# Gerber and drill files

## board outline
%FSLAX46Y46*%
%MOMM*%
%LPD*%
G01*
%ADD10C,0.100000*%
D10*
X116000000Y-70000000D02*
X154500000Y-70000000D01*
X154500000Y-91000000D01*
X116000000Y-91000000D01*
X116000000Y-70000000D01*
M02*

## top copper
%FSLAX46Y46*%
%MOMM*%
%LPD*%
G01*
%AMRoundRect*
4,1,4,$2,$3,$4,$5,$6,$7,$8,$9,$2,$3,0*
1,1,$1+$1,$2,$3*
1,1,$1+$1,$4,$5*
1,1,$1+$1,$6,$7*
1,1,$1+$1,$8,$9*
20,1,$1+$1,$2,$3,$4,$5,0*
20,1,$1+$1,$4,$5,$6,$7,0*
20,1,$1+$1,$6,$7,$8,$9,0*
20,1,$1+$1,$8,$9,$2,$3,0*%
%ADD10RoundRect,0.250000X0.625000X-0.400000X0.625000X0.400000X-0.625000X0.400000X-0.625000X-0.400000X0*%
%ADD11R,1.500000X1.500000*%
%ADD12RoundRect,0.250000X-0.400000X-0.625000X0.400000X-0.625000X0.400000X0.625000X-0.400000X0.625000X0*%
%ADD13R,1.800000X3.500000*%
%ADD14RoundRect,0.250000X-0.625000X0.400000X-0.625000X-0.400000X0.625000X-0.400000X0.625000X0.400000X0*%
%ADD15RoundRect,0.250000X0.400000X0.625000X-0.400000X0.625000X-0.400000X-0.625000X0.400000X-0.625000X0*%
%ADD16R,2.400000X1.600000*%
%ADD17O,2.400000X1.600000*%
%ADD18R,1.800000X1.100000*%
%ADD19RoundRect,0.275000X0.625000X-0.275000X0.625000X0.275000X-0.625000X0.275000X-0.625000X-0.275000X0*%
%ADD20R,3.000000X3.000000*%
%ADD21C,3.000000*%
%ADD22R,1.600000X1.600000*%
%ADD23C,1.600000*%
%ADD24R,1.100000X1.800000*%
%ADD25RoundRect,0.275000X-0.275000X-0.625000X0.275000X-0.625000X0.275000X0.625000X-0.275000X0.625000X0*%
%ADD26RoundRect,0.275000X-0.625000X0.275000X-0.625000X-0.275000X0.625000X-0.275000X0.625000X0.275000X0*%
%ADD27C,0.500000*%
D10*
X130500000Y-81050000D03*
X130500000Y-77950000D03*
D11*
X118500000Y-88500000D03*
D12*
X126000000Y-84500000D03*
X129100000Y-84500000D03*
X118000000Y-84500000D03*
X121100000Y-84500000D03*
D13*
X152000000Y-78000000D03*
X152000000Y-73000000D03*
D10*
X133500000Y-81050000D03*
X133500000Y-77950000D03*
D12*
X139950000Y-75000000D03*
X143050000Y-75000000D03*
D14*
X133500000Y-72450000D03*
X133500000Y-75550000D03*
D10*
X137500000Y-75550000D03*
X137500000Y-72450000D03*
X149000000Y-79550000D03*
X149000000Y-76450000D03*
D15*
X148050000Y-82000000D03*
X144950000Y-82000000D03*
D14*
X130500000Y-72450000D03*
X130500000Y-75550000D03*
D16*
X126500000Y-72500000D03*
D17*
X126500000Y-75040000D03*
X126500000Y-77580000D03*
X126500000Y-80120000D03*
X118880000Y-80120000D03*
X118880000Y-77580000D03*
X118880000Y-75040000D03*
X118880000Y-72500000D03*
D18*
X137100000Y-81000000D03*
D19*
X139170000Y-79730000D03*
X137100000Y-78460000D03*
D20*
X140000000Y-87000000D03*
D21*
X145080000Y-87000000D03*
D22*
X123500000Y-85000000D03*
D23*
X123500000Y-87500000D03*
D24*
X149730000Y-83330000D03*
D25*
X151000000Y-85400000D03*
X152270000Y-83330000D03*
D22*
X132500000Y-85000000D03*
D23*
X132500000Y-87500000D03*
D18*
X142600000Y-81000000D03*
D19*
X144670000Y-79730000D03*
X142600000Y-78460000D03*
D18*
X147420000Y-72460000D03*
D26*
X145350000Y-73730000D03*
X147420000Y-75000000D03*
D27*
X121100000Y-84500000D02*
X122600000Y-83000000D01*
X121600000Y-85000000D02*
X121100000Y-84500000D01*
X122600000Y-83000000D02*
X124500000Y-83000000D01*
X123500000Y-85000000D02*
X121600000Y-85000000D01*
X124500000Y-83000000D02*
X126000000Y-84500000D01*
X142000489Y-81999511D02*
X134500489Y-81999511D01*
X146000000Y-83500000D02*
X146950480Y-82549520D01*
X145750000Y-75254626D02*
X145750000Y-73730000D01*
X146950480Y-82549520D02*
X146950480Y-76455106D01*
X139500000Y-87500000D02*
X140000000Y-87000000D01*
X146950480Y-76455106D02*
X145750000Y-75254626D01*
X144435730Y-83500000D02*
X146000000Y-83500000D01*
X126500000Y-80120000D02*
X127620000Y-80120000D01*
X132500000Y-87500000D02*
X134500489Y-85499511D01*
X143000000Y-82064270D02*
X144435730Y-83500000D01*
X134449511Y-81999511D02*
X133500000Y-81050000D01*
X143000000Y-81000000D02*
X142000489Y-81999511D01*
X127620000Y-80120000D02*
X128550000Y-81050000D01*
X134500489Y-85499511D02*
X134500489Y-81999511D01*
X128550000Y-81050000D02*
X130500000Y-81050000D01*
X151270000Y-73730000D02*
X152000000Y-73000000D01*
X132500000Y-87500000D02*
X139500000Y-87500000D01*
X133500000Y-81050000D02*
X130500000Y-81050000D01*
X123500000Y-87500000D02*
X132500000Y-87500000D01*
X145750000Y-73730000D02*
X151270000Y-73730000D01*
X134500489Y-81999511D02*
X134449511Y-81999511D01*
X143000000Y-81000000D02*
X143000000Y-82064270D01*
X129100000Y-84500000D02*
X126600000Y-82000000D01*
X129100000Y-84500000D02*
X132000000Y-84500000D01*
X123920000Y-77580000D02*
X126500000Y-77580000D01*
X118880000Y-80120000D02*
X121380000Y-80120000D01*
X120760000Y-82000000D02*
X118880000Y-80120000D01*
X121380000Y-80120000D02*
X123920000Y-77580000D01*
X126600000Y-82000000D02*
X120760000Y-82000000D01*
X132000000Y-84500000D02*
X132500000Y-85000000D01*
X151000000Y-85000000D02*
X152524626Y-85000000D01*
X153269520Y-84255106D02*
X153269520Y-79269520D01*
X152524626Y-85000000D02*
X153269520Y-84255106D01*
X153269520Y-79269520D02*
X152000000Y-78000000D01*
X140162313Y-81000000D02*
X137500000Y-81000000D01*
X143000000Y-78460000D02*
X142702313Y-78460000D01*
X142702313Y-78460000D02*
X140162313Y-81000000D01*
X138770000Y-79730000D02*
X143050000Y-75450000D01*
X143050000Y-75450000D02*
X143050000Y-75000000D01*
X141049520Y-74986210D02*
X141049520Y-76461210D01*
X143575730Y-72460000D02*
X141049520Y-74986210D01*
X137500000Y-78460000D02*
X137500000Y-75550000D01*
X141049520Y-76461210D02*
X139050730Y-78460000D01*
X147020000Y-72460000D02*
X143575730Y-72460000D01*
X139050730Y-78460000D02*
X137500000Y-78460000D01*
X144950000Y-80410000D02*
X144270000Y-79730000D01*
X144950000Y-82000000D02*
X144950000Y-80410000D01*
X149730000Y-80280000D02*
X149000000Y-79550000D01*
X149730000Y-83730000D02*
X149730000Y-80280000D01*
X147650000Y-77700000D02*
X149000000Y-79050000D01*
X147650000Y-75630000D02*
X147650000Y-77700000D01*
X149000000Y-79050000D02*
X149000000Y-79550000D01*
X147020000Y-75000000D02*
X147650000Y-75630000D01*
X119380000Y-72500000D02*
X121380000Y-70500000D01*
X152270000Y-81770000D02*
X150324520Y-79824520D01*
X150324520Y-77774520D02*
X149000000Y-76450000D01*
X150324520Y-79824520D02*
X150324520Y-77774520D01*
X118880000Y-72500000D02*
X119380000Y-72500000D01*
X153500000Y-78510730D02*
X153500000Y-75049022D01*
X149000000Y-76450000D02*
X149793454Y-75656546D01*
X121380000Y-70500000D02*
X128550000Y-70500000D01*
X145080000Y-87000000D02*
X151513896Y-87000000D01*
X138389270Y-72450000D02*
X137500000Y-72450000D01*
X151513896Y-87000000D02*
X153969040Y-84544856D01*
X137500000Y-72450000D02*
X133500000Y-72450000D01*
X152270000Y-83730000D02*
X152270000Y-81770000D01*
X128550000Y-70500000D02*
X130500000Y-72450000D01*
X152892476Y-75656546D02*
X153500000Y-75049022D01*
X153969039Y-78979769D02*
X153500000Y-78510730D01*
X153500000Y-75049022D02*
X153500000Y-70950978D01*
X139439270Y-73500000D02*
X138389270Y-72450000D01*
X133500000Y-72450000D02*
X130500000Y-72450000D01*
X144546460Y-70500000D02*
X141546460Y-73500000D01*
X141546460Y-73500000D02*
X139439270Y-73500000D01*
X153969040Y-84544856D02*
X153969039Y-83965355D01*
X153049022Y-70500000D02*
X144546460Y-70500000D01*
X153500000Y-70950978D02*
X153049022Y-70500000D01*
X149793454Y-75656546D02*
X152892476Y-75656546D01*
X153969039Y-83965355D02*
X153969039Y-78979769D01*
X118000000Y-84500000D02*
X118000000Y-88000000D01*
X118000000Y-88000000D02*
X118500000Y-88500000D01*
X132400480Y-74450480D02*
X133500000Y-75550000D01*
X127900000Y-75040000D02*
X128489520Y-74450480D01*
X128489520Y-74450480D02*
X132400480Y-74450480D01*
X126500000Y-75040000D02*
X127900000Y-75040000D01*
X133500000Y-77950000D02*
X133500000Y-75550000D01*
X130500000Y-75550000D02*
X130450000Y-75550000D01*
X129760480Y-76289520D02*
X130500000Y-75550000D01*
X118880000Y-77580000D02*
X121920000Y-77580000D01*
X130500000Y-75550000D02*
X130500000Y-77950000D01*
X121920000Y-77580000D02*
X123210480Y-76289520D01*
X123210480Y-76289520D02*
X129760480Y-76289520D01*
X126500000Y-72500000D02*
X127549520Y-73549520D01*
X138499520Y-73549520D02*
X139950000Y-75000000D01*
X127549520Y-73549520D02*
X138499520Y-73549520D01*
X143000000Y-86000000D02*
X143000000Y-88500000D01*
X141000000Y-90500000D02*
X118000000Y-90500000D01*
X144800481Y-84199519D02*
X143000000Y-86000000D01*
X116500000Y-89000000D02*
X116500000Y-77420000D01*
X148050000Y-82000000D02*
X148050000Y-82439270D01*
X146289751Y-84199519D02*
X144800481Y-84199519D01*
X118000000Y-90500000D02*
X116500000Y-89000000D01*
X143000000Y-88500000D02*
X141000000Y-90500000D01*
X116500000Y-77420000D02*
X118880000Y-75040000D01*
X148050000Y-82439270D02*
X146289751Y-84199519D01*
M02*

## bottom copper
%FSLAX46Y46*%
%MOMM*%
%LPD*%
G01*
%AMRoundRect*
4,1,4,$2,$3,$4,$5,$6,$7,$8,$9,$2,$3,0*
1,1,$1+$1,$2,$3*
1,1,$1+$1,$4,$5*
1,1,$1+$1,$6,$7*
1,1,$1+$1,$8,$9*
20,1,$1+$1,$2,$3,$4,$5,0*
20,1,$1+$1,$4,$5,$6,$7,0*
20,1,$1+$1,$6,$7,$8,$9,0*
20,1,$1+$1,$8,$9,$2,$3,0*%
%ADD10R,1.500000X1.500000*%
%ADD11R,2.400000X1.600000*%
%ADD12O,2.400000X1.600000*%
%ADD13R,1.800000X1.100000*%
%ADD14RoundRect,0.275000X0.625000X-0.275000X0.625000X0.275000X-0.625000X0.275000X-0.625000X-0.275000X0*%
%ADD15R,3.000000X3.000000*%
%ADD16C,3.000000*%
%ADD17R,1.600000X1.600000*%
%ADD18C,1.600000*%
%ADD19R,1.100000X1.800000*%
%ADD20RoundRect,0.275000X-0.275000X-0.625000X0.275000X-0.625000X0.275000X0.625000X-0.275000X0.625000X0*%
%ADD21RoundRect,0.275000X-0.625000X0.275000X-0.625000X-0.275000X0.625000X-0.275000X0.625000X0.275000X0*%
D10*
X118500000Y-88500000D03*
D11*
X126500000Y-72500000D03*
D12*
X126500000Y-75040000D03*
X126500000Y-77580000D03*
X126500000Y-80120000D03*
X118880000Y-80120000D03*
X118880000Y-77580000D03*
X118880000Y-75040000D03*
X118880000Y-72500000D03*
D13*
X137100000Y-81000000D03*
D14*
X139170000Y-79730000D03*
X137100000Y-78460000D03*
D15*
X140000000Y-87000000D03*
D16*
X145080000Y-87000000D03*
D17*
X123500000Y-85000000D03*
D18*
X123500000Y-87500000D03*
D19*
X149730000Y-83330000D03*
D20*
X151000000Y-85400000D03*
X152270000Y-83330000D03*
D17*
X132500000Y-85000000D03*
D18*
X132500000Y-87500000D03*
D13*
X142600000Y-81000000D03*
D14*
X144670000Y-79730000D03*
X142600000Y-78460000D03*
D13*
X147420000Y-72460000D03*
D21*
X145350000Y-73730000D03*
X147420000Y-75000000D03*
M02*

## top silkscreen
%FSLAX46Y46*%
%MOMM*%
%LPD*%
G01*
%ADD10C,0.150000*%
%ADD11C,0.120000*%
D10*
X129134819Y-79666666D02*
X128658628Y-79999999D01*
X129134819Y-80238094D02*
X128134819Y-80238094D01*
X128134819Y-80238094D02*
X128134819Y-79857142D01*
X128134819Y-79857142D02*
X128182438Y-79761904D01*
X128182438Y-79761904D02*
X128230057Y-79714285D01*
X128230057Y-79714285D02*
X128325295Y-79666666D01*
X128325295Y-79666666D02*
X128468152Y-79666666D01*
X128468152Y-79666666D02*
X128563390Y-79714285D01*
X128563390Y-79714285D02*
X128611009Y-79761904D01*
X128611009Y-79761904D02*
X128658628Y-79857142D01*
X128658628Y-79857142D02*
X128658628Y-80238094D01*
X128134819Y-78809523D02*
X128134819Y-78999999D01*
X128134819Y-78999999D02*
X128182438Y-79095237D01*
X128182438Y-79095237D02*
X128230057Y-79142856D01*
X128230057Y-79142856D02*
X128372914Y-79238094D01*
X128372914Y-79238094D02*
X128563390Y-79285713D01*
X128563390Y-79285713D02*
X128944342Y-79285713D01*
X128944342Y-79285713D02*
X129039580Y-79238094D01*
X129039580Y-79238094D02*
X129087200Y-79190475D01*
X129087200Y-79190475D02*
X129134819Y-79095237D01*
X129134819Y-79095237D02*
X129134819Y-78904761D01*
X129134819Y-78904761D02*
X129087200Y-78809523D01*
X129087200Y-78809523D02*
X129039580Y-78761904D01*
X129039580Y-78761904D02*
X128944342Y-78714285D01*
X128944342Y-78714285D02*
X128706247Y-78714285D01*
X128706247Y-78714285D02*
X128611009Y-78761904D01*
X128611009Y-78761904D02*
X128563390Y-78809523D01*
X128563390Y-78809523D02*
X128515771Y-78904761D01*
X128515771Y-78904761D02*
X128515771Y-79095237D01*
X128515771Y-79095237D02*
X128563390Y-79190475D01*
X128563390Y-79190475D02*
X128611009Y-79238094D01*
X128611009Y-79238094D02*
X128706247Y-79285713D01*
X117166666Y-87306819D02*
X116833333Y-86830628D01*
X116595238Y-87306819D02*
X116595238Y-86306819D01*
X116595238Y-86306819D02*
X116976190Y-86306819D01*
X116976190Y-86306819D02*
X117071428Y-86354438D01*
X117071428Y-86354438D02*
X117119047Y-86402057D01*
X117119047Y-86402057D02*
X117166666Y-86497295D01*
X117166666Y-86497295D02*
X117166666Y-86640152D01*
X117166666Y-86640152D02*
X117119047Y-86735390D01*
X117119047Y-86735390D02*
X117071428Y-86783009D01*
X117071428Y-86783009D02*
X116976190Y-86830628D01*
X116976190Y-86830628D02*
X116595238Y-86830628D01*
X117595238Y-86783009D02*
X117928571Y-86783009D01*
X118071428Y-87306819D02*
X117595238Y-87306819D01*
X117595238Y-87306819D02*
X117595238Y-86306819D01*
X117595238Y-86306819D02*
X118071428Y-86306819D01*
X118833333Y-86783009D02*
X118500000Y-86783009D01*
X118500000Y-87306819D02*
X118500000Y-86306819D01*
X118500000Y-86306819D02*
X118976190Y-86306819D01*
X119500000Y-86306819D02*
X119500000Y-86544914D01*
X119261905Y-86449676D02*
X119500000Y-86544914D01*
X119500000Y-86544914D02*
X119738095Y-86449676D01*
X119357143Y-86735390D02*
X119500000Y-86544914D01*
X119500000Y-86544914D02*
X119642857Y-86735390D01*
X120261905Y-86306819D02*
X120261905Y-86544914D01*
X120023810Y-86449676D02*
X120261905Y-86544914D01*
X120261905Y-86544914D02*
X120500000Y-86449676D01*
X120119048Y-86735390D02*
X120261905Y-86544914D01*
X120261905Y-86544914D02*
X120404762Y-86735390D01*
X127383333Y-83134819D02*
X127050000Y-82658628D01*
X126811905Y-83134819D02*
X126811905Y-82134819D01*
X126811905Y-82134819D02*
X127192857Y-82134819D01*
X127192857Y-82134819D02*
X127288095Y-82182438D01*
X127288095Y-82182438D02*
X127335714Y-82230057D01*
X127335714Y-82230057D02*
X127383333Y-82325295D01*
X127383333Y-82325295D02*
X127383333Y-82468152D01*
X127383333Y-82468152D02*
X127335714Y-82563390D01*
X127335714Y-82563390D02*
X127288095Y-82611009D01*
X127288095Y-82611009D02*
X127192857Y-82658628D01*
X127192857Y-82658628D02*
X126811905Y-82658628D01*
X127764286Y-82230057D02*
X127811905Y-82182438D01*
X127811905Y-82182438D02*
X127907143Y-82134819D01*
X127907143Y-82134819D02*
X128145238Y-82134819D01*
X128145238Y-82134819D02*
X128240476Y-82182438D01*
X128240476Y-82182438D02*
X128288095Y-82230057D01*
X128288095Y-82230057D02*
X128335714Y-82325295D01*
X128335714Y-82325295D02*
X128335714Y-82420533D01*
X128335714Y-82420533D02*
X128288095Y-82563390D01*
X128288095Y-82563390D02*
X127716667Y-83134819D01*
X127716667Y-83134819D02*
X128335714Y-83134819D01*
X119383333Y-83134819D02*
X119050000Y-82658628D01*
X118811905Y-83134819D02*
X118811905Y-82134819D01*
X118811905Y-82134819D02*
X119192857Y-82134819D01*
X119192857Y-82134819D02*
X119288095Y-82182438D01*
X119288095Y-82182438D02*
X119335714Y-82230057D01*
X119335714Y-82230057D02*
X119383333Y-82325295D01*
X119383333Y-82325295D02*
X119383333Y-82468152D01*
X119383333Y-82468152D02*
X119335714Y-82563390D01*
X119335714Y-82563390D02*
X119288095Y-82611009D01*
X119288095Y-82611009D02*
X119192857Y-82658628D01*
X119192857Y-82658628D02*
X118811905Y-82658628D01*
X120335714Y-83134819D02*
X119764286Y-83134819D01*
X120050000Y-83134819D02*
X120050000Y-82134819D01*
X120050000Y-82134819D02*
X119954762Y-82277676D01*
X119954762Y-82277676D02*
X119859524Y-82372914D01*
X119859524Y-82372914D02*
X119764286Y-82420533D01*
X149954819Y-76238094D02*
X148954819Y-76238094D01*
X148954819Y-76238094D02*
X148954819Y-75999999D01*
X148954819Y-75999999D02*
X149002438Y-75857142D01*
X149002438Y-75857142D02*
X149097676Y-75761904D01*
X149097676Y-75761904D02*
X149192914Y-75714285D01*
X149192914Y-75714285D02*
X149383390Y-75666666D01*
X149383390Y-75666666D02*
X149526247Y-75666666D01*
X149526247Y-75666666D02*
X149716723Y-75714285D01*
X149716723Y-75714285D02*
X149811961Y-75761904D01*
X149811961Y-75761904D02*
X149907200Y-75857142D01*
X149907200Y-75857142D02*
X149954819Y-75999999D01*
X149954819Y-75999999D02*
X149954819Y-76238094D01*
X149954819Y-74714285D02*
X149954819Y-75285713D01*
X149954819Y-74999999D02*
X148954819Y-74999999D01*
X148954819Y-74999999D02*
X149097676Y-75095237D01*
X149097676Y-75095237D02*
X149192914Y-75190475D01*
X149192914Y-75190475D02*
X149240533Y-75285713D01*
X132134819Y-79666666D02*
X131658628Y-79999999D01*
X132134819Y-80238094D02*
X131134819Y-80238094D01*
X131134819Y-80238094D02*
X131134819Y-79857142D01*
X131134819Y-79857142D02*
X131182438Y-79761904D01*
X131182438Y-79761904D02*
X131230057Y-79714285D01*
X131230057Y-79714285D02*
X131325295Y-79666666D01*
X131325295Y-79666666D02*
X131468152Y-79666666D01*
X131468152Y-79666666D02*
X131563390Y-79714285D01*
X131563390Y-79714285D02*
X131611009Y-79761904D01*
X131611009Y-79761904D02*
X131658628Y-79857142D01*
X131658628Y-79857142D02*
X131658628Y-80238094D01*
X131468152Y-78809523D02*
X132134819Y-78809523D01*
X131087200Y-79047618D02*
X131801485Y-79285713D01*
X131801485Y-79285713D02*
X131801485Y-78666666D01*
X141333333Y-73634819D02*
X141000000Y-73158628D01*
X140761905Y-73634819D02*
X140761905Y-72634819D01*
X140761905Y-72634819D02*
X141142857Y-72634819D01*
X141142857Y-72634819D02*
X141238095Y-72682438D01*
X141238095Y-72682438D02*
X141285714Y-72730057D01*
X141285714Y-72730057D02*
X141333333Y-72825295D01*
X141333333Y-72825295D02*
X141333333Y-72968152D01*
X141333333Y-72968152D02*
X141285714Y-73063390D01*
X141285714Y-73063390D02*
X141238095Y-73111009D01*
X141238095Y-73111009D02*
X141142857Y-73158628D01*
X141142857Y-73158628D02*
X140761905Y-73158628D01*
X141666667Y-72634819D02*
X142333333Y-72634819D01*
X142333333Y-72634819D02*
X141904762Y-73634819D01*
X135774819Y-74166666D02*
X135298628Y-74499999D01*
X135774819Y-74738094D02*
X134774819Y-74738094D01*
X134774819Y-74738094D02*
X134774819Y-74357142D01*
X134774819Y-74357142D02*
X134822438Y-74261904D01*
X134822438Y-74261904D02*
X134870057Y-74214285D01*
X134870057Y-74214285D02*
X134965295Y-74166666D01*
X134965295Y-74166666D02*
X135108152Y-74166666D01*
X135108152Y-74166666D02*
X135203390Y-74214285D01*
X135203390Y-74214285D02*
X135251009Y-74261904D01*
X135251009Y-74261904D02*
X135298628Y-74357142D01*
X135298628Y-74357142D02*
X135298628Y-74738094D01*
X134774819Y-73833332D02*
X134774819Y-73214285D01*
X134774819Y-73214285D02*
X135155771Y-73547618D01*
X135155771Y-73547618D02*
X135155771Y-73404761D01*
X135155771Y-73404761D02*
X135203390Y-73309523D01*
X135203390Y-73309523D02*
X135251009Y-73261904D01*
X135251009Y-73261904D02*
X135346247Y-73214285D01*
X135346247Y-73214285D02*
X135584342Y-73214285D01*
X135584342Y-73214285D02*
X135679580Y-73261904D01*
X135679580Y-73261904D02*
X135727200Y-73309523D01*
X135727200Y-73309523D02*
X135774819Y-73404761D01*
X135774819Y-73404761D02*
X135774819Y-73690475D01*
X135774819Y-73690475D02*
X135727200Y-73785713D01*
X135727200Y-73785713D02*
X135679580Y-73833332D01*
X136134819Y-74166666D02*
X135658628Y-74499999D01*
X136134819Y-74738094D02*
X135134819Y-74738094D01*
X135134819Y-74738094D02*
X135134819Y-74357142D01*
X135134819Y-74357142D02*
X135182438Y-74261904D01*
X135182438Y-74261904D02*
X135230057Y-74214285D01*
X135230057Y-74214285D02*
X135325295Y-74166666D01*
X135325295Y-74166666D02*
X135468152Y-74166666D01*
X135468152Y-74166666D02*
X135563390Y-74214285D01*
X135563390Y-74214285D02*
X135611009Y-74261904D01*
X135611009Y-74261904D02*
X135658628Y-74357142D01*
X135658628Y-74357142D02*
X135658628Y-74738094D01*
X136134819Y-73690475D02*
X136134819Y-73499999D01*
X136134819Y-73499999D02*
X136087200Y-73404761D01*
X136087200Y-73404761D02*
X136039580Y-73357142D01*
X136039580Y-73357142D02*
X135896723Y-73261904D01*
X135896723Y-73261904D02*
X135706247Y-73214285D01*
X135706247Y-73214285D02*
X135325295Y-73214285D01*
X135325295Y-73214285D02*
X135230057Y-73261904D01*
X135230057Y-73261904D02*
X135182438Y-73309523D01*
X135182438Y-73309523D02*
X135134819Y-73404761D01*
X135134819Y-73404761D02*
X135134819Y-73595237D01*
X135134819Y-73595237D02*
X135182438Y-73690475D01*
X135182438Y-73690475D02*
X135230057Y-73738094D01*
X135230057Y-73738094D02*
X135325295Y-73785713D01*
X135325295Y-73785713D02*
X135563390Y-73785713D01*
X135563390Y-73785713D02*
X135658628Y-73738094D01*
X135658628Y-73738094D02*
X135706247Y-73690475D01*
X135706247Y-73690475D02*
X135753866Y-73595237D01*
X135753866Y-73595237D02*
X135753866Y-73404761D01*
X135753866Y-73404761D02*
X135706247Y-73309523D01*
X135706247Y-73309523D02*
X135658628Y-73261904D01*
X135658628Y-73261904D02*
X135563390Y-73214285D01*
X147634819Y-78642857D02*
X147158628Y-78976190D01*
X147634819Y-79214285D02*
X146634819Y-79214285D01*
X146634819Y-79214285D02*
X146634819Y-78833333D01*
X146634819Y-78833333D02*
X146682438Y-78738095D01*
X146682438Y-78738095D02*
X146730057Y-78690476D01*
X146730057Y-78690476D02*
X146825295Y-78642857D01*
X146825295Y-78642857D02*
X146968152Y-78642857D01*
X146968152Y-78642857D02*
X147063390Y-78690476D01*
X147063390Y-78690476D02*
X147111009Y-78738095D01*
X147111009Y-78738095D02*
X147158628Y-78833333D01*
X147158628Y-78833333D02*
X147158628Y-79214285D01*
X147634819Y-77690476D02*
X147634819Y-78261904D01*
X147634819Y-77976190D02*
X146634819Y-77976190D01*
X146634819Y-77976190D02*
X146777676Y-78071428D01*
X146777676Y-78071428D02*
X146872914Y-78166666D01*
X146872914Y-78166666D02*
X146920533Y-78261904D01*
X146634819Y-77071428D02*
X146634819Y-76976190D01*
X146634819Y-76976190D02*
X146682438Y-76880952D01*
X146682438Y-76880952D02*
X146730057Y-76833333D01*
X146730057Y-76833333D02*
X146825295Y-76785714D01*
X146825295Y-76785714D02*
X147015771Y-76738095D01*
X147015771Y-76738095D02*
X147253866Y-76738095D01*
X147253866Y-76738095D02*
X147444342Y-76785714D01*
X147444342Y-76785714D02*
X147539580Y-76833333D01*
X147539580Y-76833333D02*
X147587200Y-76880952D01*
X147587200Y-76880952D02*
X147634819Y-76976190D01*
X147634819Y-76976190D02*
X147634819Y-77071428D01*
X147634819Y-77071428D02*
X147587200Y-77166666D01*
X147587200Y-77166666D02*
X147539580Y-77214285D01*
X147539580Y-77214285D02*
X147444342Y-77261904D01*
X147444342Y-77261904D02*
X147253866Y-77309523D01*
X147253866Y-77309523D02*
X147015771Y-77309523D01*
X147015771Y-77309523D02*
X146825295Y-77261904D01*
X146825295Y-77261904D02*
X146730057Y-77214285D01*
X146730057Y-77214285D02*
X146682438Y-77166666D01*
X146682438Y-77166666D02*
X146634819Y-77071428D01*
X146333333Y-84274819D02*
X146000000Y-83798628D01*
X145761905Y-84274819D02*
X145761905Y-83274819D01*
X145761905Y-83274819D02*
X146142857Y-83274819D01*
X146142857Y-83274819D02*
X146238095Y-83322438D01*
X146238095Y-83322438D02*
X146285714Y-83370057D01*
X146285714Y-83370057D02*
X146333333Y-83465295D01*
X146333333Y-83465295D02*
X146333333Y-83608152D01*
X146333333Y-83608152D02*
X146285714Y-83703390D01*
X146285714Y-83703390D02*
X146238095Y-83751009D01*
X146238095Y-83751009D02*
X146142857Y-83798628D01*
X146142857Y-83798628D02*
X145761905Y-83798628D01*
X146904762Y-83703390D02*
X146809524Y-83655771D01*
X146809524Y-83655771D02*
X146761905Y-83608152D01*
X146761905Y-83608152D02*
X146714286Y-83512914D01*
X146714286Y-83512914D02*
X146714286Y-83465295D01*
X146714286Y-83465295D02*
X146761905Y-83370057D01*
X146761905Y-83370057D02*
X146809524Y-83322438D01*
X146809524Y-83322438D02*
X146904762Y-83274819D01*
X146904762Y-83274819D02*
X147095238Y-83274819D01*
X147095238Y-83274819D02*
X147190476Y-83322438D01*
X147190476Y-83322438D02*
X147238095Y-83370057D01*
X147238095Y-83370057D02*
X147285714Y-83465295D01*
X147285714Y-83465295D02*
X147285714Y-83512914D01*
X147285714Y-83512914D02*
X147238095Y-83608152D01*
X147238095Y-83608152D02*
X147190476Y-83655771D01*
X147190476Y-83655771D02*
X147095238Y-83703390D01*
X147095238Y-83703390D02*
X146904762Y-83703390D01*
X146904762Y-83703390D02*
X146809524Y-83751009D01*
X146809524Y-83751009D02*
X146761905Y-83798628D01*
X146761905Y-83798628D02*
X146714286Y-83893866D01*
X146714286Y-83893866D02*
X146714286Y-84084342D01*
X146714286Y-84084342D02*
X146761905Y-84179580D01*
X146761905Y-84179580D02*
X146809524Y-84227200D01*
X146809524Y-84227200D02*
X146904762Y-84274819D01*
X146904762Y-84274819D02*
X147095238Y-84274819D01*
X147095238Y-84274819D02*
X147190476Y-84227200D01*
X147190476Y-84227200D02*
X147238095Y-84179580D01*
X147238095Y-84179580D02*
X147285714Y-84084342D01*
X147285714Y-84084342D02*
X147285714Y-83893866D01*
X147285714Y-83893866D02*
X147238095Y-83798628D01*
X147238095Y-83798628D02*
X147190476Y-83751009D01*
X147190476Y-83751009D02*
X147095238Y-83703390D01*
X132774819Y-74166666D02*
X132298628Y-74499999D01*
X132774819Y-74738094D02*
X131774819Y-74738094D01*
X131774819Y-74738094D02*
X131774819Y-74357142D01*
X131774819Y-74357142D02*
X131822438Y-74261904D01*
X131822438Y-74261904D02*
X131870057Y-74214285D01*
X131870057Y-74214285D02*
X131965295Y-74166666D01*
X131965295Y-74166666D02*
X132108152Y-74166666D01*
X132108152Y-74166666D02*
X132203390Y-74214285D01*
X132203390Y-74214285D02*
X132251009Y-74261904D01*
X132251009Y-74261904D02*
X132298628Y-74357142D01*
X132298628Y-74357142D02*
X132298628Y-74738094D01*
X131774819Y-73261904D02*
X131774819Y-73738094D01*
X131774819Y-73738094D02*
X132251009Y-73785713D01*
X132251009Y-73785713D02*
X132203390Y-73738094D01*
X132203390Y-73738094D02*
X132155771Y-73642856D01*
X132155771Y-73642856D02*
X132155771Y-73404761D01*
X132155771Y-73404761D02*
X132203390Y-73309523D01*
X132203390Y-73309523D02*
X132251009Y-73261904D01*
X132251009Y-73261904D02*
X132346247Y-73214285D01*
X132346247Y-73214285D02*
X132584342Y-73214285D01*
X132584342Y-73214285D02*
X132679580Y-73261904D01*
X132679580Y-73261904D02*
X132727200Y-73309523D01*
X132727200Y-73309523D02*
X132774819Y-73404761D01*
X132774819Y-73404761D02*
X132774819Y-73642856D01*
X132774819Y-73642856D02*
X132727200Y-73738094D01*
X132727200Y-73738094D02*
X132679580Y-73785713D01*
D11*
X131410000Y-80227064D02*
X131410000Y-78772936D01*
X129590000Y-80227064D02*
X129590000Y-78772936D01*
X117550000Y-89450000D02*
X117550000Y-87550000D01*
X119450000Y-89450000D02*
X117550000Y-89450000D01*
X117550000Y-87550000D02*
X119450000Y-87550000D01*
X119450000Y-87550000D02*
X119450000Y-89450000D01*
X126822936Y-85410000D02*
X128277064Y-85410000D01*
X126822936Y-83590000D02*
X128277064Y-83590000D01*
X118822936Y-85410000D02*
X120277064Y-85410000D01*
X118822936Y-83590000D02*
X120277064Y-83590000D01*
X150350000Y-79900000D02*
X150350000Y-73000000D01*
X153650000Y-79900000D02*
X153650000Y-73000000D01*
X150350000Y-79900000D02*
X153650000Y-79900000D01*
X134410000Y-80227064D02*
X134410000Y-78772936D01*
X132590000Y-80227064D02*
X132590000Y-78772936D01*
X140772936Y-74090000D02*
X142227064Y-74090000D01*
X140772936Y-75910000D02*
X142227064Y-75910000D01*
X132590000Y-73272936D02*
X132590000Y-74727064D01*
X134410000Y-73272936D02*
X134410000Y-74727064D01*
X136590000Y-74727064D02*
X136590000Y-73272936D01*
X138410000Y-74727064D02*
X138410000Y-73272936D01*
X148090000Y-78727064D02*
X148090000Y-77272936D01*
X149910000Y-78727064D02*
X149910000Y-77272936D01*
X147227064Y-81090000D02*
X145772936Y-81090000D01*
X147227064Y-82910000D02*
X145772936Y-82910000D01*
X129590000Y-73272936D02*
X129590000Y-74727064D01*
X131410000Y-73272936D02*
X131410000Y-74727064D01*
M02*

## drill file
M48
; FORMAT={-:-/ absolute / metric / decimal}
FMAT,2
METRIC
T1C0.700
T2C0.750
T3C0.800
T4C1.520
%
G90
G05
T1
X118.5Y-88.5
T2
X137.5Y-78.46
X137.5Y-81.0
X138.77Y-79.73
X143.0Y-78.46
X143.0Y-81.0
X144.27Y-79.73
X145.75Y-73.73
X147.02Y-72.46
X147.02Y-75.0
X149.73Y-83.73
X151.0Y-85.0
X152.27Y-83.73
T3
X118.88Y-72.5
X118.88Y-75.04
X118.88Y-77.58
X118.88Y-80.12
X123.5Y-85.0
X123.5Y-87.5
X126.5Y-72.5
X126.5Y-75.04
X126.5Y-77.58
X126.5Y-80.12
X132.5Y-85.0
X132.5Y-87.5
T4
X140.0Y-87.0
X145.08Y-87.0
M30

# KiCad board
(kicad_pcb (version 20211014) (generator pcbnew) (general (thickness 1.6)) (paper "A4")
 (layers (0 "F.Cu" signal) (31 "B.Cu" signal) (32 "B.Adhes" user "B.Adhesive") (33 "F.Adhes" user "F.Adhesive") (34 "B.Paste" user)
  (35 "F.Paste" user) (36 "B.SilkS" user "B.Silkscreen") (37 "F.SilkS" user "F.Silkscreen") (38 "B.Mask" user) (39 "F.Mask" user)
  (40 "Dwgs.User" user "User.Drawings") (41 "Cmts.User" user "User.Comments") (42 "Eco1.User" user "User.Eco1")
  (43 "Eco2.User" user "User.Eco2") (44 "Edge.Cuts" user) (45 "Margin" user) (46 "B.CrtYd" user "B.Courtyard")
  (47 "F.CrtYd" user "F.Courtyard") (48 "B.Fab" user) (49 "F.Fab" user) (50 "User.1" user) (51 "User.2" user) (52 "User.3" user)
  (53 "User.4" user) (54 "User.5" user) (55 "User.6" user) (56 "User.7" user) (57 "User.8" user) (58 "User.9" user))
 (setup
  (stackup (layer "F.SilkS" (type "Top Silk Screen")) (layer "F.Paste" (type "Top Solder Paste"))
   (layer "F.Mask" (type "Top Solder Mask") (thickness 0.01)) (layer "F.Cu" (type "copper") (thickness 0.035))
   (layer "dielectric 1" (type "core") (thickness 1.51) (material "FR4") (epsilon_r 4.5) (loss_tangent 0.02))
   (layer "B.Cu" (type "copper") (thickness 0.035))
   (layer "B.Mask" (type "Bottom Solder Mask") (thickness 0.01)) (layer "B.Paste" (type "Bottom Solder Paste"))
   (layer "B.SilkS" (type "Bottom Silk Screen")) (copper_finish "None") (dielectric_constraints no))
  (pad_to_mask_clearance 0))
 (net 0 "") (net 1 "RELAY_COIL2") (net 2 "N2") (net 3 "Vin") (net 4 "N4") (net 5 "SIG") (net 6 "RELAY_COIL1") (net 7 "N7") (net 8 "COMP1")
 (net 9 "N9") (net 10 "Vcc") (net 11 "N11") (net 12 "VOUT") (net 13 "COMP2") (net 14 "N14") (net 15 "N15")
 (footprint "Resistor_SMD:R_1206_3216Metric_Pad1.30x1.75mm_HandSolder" (layer "F.Cu") (at 130.5 79.5 90)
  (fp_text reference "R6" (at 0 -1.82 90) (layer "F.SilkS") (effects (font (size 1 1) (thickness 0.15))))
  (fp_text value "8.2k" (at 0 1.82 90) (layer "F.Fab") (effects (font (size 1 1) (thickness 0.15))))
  (fp_line (start -0.727064 0.91) (end 0.727064 0.91) (layer "F.SilkS") (width 0.12))
  (fp_line (start -0.727064 -0.91) (end 0.727064 -0.91) (layer "F.SilkS") (width 0.12))
  (pad "1" smd roundrect (at -1.55 0 90) (size 1.3 1.75) (layers "F.Cu" "F.Paste" "F.Mask") (roundrect_rratio 0.1923076923)
   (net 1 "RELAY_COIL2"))
  (pad "2" smd roundrect (at 1.55 0 90) (size 1.3 1.75) (layers "F.Cu" "F.Paste" "F.Mask") (roundrect_rratio 0.1923076923) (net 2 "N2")))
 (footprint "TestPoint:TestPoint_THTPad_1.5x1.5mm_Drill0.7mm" (layer "F.Cu") (at 118.5 88.5)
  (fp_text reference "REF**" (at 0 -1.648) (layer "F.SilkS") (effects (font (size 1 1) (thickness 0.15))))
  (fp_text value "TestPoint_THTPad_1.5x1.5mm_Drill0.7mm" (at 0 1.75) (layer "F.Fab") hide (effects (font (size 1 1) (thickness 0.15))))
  (fp_line (start -0.95 0.95) (end -0.95 -0.95) (layer "F.SilkS") (width 0.12))
  (fp_line (start 0.95 0.95) (end -0.95 0.95) (layer "F.SilkS") (width 0.12))
  (fp_line (start -0.95 -0.95) (end 0.95 -0.95) (layer "F.SilkS") (width 0.12))
  (fp_line (start 0.95 -0.95) (end 0.95 0.95) (layer "F.SilkS") (width 0.12))
  (pad "1" thru_hole rect (at 0 0) (size 1.5 1.5) (drill 0.7) (layers *.Cu *.Mask) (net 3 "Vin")))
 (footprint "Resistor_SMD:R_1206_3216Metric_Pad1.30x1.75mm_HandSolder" (layer "F.Cu") (at 127.55 84.5)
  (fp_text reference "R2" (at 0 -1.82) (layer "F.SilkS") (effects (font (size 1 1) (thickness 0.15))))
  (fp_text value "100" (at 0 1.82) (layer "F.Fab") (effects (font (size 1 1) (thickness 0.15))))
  (fp_line (start -0.727064 0.91) (end 0.727064 0.91) (layer "F.SilkS") (width 0.12))
  (fp_line (start -0.727064 -0.91) (end 0.727064 -0.91) (layer "F.SilkS") (width 0.12))
  (pad "1" smd roundrect (at -1.55 0) (size 1.3 1.75) (layers "F.Cu" "F.Paste" "F.Mask") (roundrect_rratio 0.1923076923) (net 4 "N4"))
  (pad "2" smd roundrect (at 1.55 0) (size 1.3 1.75) (layers "F.Cu" "F.Paste" "F.Mask") (roundrect_rratio 0.1923076923) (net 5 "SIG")))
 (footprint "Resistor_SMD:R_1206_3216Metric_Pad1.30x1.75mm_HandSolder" (layer "F.Cu") (at 119.55 84.5)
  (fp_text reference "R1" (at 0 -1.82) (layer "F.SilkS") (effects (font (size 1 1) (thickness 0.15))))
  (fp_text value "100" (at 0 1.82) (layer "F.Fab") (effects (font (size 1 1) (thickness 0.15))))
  (fp_line (start -0.727064 0.91) (end 0.727064 0.91) (layer "F.SilkS") (width 0.12))
  (fp_line (start -0.727064 -0.91) (end 0.727064 -0.91) (layer "F.SilkS") (width 0.12))
  (pad "1" smd roundrect (at -1.55 0) (size 1.3 1.75) (layers "F.Cu" "F.Paste" "F.Mask") (roundrect_rratio 0.1923076923) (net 3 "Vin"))
  (pad "2" smd roundrect (at 1.55 0) (size 1.3 1.75) (layers "F.Cu" "F.Paste" "F.Mask") (roundrect_rratio 0.1923076923) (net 4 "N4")))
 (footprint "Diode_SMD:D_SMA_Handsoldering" (layer "F.Cu") (at 152 75.5 90)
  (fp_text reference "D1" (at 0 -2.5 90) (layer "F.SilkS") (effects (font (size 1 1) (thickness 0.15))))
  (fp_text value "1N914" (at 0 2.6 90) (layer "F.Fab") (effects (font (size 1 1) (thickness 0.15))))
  (fp_line (start -4.4 -1.65) (end 2.5 -1.65) (layer "F.SilkS") (width 0.12))
  (fp_line (start -4.4 1.65) (end 2.5 1.65) (layer "F.SilkS") (width 0.12))
  (fp_line (start -4.4 -1.65) (end -4.4 1.65) (layer "F.SilkS") (width 0.12))
  (pad "1" smd rect (at -2.5 0 90) (size 3.5 1.8) (layers "F.Cu" "F.Paste" "F.Mask") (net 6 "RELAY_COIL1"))
  (pad "2" smd rect (at 2.5 0 90) (size 3.5 1.8) (layers "F.Cu" "F.Paste" "F.Mask") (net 1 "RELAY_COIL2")))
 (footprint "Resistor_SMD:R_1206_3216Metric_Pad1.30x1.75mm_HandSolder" (layer "F.Cu") (at 133.5 79.5 90)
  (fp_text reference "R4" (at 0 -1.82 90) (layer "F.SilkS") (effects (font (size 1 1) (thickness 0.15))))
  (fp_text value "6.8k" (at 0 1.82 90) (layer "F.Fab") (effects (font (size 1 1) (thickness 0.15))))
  (fp_line (start -0.727064 0.91) (end 0.727064 0.91) (layer "F.SilkS") (width 0.12))
  (fp_line (start -0.727064 -0.91) (end 0.727064 -0.91) (layer "F.SilkS") (width 0.12))
  (pad "1" smd roundrect (at -1.55 0 90) (size 1.3 1.75) (layers "F.Cu" "F.Paste" "F.Mask") (roundrect_rratio 0.1923076923)
   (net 1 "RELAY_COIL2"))
  (pad "2" smd roundrect (at 1.55 0 90) (size 1.3 1.75) (layers "F.Cu" "F.Paste" "F.Mask") (roundrect_rratio 0.1923076923) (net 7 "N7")))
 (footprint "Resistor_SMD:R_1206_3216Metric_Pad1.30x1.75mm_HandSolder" (layer "F.Cu") (at 141.5 75)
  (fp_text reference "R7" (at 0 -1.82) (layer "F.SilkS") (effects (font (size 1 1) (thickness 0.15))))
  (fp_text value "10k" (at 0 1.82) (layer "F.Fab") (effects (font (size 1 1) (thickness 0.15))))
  (fp_line (start -0.727064 -0.91) (end 0.727064 -0.91) (layer "F.SilkS") (width 0.12))
  (fp_line (start -0.727064 0.91) (end 0.727064 0.91) (layer "F.SilkS") (width 0.12))
  (pad "1" smd roundrect (at -1.55 0) (size 1.3 1.75) (layers "F.Cu" "F.Paste" "F.Mask") (roundrect_rratio 0.1923076923) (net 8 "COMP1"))
  (pad "2" smd roundrect (at 1.55 0) (size 1.3 1.75) (layers "F.Cu" "F.Paste" "F.Mask") (roundrect_rratio 0.1923076923) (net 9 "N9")))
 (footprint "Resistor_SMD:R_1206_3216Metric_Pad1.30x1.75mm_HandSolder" (layer "F.Cu") (at 133.5 74 -90)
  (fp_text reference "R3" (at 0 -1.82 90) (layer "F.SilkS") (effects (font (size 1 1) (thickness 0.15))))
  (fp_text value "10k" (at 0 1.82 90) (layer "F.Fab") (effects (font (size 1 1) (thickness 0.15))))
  (fp_line (start -0.727064 0.91) (end 0.727064 0.91) (layer "F.SilkS") (width 0.12))
  (fp_line (start -0.727064 -0.91) (end 0.727064 -0.91) (layer "F.SilkS") (width 0.12))
  (pad "1" smd roundrect (at -1.55 0 270) (size 1.3 1.75) (layers "F.Cu" "F.Paste" "F.Mask") (roundrect_rratio 0.1923076923) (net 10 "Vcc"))
  (pad "2" smd roundrect (at 1.55 0 270) (size 1.3 1.75) (layers "F.Cu" "F.Paste" "F.Mask") (roundrect_rratio 0.1923076923) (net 7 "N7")))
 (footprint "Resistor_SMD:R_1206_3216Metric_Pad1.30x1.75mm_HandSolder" (layer "F.Cu") (at 137.5 74 90)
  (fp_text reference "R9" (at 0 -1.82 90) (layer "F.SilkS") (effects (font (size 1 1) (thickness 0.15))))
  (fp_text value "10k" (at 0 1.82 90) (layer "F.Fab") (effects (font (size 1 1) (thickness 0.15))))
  (fp_line (start -0.727064 -0.91) (end 0.727064 -0.91) (layer "F.SilkS") (width 0.12))
  (fp_line (start -0.727064 0.91) (end 0.727064 0.91) (layer "F.SilkS") (width 0.12))
  (pad "1" smd roundrect (at -1.55 0 90) (size 1.3 1.75) (layers "F.Cu" "F.Paste" "F.Mask") (roundrect_rratio 0.1923076923) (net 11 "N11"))
  (pad "2" smd roundrect (at 1.55 0 90) (size 1.3 1.75) (layers "F.Cu" "F.Paste" "F.Mask") (roundrect_rratio 0.1923076923) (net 10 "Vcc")))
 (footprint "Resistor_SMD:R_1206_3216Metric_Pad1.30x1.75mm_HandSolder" (layer "F.Cu") (at 149 78 90)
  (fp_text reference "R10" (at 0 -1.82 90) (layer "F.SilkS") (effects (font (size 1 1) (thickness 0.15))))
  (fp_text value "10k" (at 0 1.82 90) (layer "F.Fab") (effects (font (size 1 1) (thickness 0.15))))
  (fp_line (start -0.727064 -0.91) (end 0.727064 -0.91) (layer "F.SilkS") (width 0.12))
  (fp_line (start -0.727064 0.91) (end 0.727064 0.91) (layer "F.SilkS") (width 0.12))
  (pad "1" smd roundrect (at -1.55 0 90) (size 1.3 1.75) (layers "F.Cu" "F.Paste" "F.Mask") (roundrect_rratio 0.1923076923) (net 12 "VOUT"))
  (pad "2" smd roundrect (at 1.55 0 90) (size 1.3 1.75) (layers "F.Cu" "F.Paste" "F.Mask") (roundrect_rratio 0.1923076923) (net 10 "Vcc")))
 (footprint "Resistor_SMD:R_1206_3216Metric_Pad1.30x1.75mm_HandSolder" (layer "F.Cu") (at 146.5 82 180)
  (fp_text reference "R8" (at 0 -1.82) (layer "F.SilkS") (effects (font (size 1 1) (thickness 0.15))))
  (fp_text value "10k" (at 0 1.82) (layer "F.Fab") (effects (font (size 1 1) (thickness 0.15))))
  (fp_line (start -0.727064 0.91) (end 0.727064 0.91) (layer "F.SilkS") (width 0.12))
  (fp_line (start -0.727064 -0.91) (end 0.727064 -0.91) (layer "F.SilkS") (width 0.12))
  (pad "1" smd roundrect (at -1.55 0 180) (size 1.3 1.75) (layers "F.Cu" "F.Paste" "F.Mask") (roundrect_rratio 0.1923076923)
   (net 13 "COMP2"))
  (pad "2" smd roundrect (at 1.55 0 180) (size 1.3 1.75) (layers "F.Cu" "F.Paste" "F.Mask") (roundrect_rratio 0.1923076923) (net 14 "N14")))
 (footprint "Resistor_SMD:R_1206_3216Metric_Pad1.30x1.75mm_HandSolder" (layer "F.Cu") (at 130.5 74 -90)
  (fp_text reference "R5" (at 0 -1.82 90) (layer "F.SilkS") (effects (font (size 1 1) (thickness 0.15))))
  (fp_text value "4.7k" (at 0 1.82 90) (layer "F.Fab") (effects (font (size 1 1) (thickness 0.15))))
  (fp_line (start -0.727064 0.91) (end 0.727064 0.91) (layer "F.SilkS") (width 0.12))
  (fp_line (start -0.727064 -0.91) (end 0.727064 -0.91) (layer "F.SilkS") (width 0.12))
  (pad "1" smd roundrect (at -1.55 0 270) (size 1.3 1.75) (layers "F.Cu" "F.Paste" "F.Mask") (roundrect_rratio 0.1923076923) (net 10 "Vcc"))
  (pad "2" smd roundrect (at 1.55 0 270) (size 1.3 1.75) (layers "F.Cu" "F.Paste" "F.Mask") (roundrect_rratio 0.1923076923) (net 2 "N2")))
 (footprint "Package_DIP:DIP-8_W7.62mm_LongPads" (layer "B.Cu") (at 126.5 72.5 180)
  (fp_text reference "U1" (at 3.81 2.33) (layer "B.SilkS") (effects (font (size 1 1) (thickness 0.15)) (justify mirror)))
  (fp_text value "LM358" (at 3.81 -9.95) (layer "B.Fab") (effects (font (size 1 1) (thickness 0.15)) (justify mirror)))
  (pad "1" thru_hole rect (at 0 0 180) (size 2.4 1.6) (drill 0.8) (layers *.Cu *.Mask) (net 8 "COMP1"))
  (pad "2" thru_hole oval (at 0 -2.54 180) (size 2.4 1.6) (drill 0.8) (layers *.Cu *.Mask) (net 7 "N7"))
  (pad "3" thru_hole oval (at 0 -5.08 180) (size 2.4 1.6) (drill 0.8) (layers *.Cu *.Mask) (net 5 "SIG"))
  (pad "4" thru_hole oval (at 0 -7.62 180) (size 2.4 1.6) (drill 0.8) (layers *.Cu *.Mask) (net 1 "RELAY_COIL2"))
  (pad "5" thru_hole oval (at 7.62 -7.62 180) (size 2.4 1.6) (drill 0.8) (layers *.Cu *.Mask) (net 5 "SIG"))
  (pad "6" thru_hole oval (at 7.62 -5.08 180) (size 2.4 1.6) (drill 0.8) (layers *.Cu *.Mask) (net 2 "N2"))
  (pad "7" thru_hole oval (at 7.62 -2.54 180) (size 2.4 1.6) (drill 0.8) (layers *.Cu *.Mask) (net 13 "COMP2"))
  (pad "8" thru_hole oval (at 7.62 0 180) (size 2.4 1.6) (drill 0.8) (layers *.Cu *.Mask) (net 10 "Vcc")))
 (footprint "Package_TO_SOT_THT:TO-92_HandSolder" (layer "B.Cu") (at 137.5 81 90)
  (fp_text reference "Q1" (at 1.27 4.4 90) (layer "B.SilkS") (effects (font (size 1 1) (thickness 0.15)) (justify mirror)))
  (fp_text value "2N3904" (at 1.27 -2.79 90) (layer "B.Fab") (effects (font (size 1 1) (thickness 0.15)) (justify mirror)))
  (pad "1" thru_hole rect (at 0 0 90) (size 1.1 1.8) (drill 0.75 (offset 0 -0.4)) (layers *.Cu *.Mask) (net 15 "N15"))
  (pad "2" thru_hole roundrect (at 1.27 1.27 90) (size 1.1 1.8) (drill 0.75 (offset 0 0.4)) (layers *.Cu *.Mask) (roundrect_rratio 0.25)
   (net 9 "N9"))
  (pad "3" thru_hole roundrect (at 2.54 0 90) (size 1.1 1.8) (drill 0.75 (offset 0 -0.4)) (layers *.Cu *.Mask) (roundrect_rratio 0.25)
   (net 11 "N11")))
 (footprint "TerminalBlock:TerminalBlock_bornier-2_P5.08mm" (layer "B.Cu") (at 140 87)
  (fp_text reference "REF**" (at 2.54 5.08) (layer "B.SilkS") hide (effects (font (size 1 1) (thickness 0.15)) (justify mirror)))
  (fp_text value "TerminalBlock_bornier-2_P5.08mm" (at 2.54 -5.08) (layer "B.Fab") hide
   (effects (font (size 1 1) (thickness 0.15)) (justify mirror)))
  (pad "1" thru_hole rect (at 0 0) (size 3 3) (drill 1.52) (layers *.Cu *.Mask) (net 1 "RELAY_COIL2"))
  (pad "2" thru_hole circle (at 5.08 0) (size 3 3) (drill 1.52) (layers *.Cu *.Mask) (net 10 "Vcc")))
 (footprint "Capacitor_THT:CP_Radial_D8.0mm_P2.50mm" (layer "B.Cu") (at 123.5 85 -90)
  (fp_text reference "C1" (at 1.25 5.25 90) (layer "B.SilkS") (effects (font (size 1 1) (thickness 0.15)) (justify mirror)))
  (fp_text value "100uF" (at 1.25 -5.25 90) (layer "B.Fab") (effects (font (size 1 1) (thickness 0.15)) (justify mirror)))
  (pad "1" thru_hole rect (at 0 0 270) (size 1.6 1.6) (drill 0.8) (layers *.Cu *.Mask) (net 4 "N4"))
  (pad "2" thru_hole circle (at 2.5 0 270) (size 1.6 1.6) (drill 0.8) (layers *.Cu *.Mask) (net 1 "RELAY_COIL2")))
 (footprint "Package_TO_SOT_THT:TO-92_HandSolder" (layer "B.Cu") (at 149.73 83.73)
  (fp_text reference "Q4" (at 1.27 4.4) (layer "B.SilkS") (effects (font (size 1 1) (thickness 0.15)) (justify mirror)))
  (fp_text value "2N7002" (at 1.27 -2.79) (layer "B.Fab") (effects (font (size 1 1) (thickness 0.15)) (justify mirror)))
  (pad "1" thru_hole rect (at 0 0) (size 1.1 1.8) (drill 0.75 (offset 0 -0.4)) (layers *.Cu *.Mask) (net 12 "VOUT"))
  (pad "2" thru_hole roundrect (at 1.27 1.27) (size 1.1 1.8) (drill 0.75 (offset 0 0.4)) (layers *.Cu *.Mask) (roundrect_rratio 0.25)
   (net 6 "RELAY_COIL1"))
  (pad "3" thru_hole roundrect (at 2.54 0) (size 1.1 1.8) (drill 0.75 (offset 0 -0.4)) (layers *.Cu *.Mask) (roundrect_rratio 0.25)
   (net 10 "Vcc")))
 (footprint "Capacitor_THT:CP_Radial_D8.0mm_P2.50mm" (layer "B.Cu") (at 132.5 85 -90)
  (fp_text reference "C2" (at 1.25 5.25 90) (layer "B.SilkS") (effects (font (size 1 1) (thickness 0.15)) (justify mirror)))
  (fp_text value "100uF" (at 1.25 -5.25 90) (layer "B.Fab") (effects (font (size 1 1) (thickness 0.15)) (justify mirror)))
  (pad "1" thru_hole rect (at 0 0 270) (size 1.6 1.6) (drill 0.8) (layers *.Cu *.Mask) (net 5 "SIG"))
  (pad "2" thru_hole circle (at 2.5 0 270) (size 1.6 1.6) (drill 0.8) (layers *.Cu *.Mask) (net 1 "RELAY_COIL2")))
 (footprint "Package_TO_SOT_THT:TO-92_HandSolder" (layer "B.Cu") (at 143 81 90)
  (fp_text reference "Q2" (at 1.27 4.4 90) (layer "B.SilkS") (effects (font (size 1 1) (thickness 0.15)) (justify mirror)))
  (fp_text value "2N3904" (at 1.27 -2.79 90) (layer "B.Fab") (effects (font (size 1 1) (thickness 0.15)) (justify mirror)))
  (pad "1" thru_hole rect (at 0 0 90) (size 1.1 1.8) (drill 0.75 (offset 0 -0.4)) (layers *.Cu *.Mask) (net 1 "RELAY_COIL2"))
  (pad "2" thru_hole roundrect (at 1.27 1.27 90) (size 1.1 1.8) (drill 0.75 (offset 0 0.4)) (layers *.Cu *.Mask) (roundrect_rratio 0.25)
   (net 14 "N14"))
  (pad "3" thru_hole roundrect (at 2.54 0 90) (size 1.1 1.8) (drill 0.75 (offset 0 -0.4)) (layers *.Cu *.Mask) (roundrect_rratio 0.25)
   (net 15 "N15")))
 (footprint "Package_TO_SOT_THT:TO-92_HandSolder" (layer "B.Cu") (at 147.02 72.46 -90)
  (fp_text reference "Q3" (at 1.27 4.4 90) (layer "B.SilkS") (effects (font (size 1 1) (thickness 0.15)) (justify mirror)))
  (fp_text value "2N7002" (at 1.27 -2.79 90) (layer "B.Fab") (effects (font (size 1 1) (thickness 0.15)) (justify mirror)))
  (pad "1" thru_hole rect (at 0 0 270) (size 1.1 1.8) (drill 0.75 (offset 0 -0.4)) (layers *.Cu *.Mask) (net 11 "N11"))
  (pad "2" thru_hole roundrect (at 1.27 1.27 270) (size 1.1 1.8) (drill 0.75 (offset 0 0.4)) (layers *.Cu *.Mask) (roundrect_rratio 0.25)
   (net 1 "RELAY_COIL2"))
  (pad "3" thru_hole roundrect (at 2.54 0 270) (size 1.1 1.8) (drill 0.75 (offset 0 -0.4)) (layers *.Cu *.Mask) (roundrect_rratio 0.25)
   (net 12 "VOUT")))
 (gr_rect (start 154.5 70) (end 116 91) (layer "Edge.Cuts") (width 0.1) (fill none))
 (segment (start 121.1 84.5) (end 122.6 83) (width 0.5) (layer "F.Cu") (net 4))
 (segment (start 121.6 85) (end 121.1 84.5) (width 0.5) (layer "F.Cu") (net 4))
 (segment (start 122.6 83) (end 124.5 83) (width 0.5) (layer "F.Cu") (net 4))
 (segment (start 123.5 85) (end 121.6 85) (width 0.5) (layer "F.Cu") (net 4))
 (segment (start 124.5 83) (end 126 84.5) (width 0.5) (layer "F.Cu") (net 4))
 (segment (start 142.000489 81.999511) (end 134.500489 81.999511) (width 0.5) (layer "F.Cu") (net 1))
 (segment (start 146 83.5) (end 146.95048 82.54952) (width 0.5) (layer "F.Cu") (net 1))
 (segment (start 145.75 75.254626) (end 145.75 73.73) (width 0.5) (layer "F.Cu") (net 1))
 (segment (start 146.95048 82.54952) (end 146.95048 76.455106) (width 0.5) (layer "F.Cu") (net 1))
 (segment (start 139.5 87.5) (end 140 87) (width 0.5) (layer "F.Cu") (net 1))
 (segment (start 146.95048 76.455106) (end 145.75 75.254626) (width 0.5) (layer "F.Cu") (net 1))
 (segment (start 144.43573 83.5) (end 146 83.5) (width 0.5) (layer "F.Cu") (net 1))
 (segment (start 126.5 80.12) (end 127.62 80.12) (width 0.5) (layer "F.Cu") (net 1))
 (segment (start 132.5 87.5) (end 134.500489 85.499511) (width 0.5) (layer "F.Cu") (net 1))
 (segment (start 143 82.06427) (end 144.43573 83.5) (width 0.5) (layer "F.Cu") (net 1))
 (segment (start 134.449511 81.999511) (end 133.5 81.05) (width 0.5) (layer "F.Cu") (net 1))
 (segment (start 143 81) (end 142.000489 81.999511) (width 0.5) (layer "F.Cu") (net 1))
 (segment (start 127.62 80.12) (end 128.55 81.05) (width 0.5) (layer "F.Cu") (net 1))
 (segment (start 134.500489 85.499511) (end 134.500489 81.999511) (width 0.5) (layer "F.Cu") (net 1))
 (segment (start 128.55 81.05) (end 130.5 81.05) (width 0.5) (layer "F.Cu") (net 1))
 (segment (start 151.27 73.73) (end 152 73) (width 0.5) (layer "F.Cu") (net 1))
 (segment (start 132.5 87.5) (end 139.5 87.5) (width 0.5) (layer "F.Cu") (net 1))
 (segment (start 133.5 81.05) (end 130.5 81.05) (width 0.5) (layer "F.Cu") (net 1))
 (segment (start 123.5 87.5) (end 132.5 87.5) (width 0.5) (layer "F.Cu") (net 1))
 (segment (start 145.75 73.73) (end 151.27 73.73) (width 0.5) (layer "F.Cu") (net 1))
 (segment (start 134.500489 81.999511) (end 134.449511 81.999511) (width 0.5) (layer "F.Cu") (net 1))
 (segment (start 143 81) (end 143 82.06427) (width 0.5) (layer "F.Cu") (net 1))
 (segment (start 129.1 84.5) (end 126.6 82) (width 0.5) (layer "F.Cu") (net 5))
 (segment (start 129.1 84.5) (end 132 84.5) (width 0.5) (layer "F.Cu") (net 5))
 (segment (start 123.92 77.58) (end 126.5 77.58) (width 0.5) (layer "F.Cu") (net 5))
 (segment (start 118.88 80.12) (end 121.38 80.12) (width 0.5) (layer "F.Cu") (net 5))
 (segment (start 120.76 82) (end 118.88 80.12) (width 0.5) (layer "F.Cu") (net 5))
 (segment (start 121.38 80.12) (end 123.92 77.58) (width 0.5) (layer "F.Cu") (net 5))
 (segment (start 126.6 82) (end 120.76 82) (width 0.5) (layer "F.Cu") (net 5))
 (segment (start 132 84.5) (end 132.5 85) (width 0.5) (layer "F.Cu") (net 5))
 (segment (start 151 85) (end 152.524626 85) (width 0.5) (layer "F.Cu") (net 6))
 (segment (start 153.26952 84.255106) (end 153.26952 79.26952) (width 0.5) (layer "F.Cu") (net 6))
 (segment (start 152.524626 85) (end 153.26952 84.255106) (width 0.5) (layer "F.Cu") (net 6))
 (segment (start 153.26952 79.26952) (end 152 78) (width 0.5) (layer "F.Cu") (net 6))
 (segment (start 140.162313 81) (end 137.5 81) (width 0.5) (layer "F.Cu") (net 15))
 (segment (start 143 78.46) (end 142.702313 78.46) (width 0.5) (layer "F.Cu") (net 15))
 (segment (start 142.702313 78.46) (end 140.162313 81) (width 0.5) (layer "F.Cu") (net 15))
 (segment (start 138.77 79.73) (end 143.05 75.45) (width 0.5) (layer "F.Cu") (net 9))
 (segment (start 143.05 75.45) (end 143.05 75) (width 0.5) (layer "F.Cu") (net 9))
 (segment (start 141.04952 74.98621) (end 141.04952 76.46121) (width 0.5) (layer "F.Cu") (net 11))
 (segment (start 143.57573 72.46) (end 141.04952 74.98621) (width 0.5) (layer "F.Cu") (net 11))
 (segment (start 137.5 78.46) (end 137.5 75.55) (width 0.5) (layer "F.Cu") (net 11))
 (segment (start 141.04952 76.46121) (end 139.05073 78.46) (width 0.5) (layer "F.Cu") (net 11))
 (segment (start 147.02 72.46) (end 143.57573 72.46) (width 0.5) (layer "F.Cu") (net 11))
 (segment (start 139.05073 78.46) (end 137.5 78.46) (width 0.5) (layer "F.Cu") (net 11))
 (segment (start 144.95 80.41) (end 144.27 79.73) (width 0.5) (layer "F.Cu") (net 14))
 (segment (start 144.95 82) (end 144.95 80.41) (width 0.5) (layer "F.Cu") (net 14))
 (segment (start 149.73 80.28) (end 149 79.55) (width 0.5) (layer "F.Cu") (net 12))
 (segment (start 149.73 83.73) (end 149.73 80.28) (width 0.5) (layer "F.Cu") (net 12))
 (segment (start 147.65 77.7) (end 149 79.05) (width 0.5) (layer "F.Cu") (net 12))
 (segment (start 147.65 75.63) (end 147.65 77.7) (width 0.5) (layer "F.Cu") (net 12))
 (segment (start 149 79.05) (end 149 79.55) (width 0.5) (layer "F.Cu") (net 12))
 (segment (start 147.02 75) (end 147.65 75.63) (width 0.5) (layer "F.Cu") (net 12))
 (segment (start 119.38 72.5) (end 121.38 70.5) (width 0.5) (layer "F.Cu") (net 10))
 (segment (start 152.27 81.77) (end 150.32452 79.82452) (width 0.5) (layer "F.Cu") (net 10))
 (segment (start 150.32452 77.77452) (end 149 76.45) (width 0.5) (layer "F.Cu") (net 10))
 (segment (start 150.32452 79.82452) (end 150.32452 77.77452) (width 0.5) (layer "F.Cu") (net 10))
 (segment (start 118.88 72.5) (end 119.38 72.5) (width 0.5) (layer "F.Cu") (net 10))
 (segment (start 153.5 78.51073) (end 153.5 75.049022) (width 0.5) (layer "F.Cu") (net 10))
 (segment (start 149 76.45) (end 149.793454 75.656546) (width 0.5) (layer "F.Cu") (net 10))
 (segment (start 121.38 70.5) (end 128.55 70.5) (width 0.5) (layer "F.Cu") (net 10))
 (segment (start 145.08 87) (end 151.513896 87) (width 0.5) (layer "F.Cu") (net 10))
 (segment (start 138.38927 72.45) (end 137.5 72.45) (width 0.5) (layer "F.Cu") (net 10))
 (segment (start 151.513896 87) (end 153.96904 84.544856) (width 0.5) (layer "F.Cu") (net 10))
 (segment (start 137.5 72.45) (end 133.5 72.45) (width 0.5) (layer "F.Cu") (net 10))
 (segment (start 152.27 83.73) (end 152.27 81.77) (width 0.5) (layer "F.Cu") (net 10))
 (segment (start 128.55 70.5) (end 130.5 72.45) (width 0.5) (layer "F.Cu") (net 10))
 (segment (start 152.892476 75.656546) (end 153.5 75.049022) (width 0.5) (layer "F.Cu") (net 10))
 (segment (start 153.969039 78.979769) (end 153.5 78.51073) (width 0.5) (layer "F.Cu") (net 10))
 (segment (start 153.5 75.049022) (end 153.5 70.950978) (width 0.5) (layer "F.Cu") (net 10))
 (segment (start 139.43927 73.5) (end 138.38927 72.45) (width 0.5) (layer "F.Cu") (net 10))
 (segment (start 133.5 72.45) (end 130.5 72.45) (width 0.5) (layer "F.Cu") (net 10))
 (segment (start 144.54646 70.5) (end 141.54646 73.5) (width 0.5) (layer "F.Cu") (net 10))
 (segment (start 141.54646 73.5) (end 139.43927 73.5) (width 0.5) (layer "F.Cu") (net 10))
 (segment (start 153.96904 84.544856) (end 153.969039 83.965355) (width 0.5) (layer "F.Cu") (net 10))
 (segment (start 153.049022 70.5) (end 144.54646 70.5) (width 0.5) (layer "F.Cu") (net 10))
 (segment (start 153.5 70.950978) (end 153.049022 70.5) (width 0.5) (layer "F.Cu") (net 10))
 (segment (start 149.793454 75.656546) (end 152.892476 75.656546) (width 0.5) (layer "F.Cu") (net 10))
 (segment (start 153.969039 83.965355) (end 153.969039 78.979769) (width 0.5) (layer "F.Cu") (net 10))
 (segment (start 118 84.5) (end 118 88) (width 0.5) (layer "F.Cu") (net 3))
 (segment (start 118 88) (end 118.5 88.5) (width 0.5) (layer "F.Cu") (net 3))
 (segment (start 132.40048 74.45048) (end 133.5 75.55) (width 0.5) (layer "F.Cu") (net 7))
 (segment (start 127.9 75.04) (end 128.48952 74.45048) (width 0.5) (layer "F.Cu") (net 7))
 (segment (start 128.48952 74.45048) (end 132.40048 74.45048) (width 0.5) (layer "F.Cu") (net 7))
 (segment (start 126.5 75.04) (end 127.9 75.04) (width 0.5) (layer "F.Cu") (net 7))
 (segment (start 133.5 77.95) (end 133.5 75.55) (width 0.5) (layer "F.Cu") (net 7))
 (segment (start 130.5 75.55) (end 130.45 75.55) (width 0.5) (layer "F.Cu") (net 2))
 (segment (start 129.76048 76.28952) (end 130.5 75.55) (width 0.5) (layer "F.Cu") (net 2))
 (segment (start 118.88 77.58) (end 121.92 77.58) (width 0.5) (layer "F.Cu") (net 2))
 (segment (start 130.5 75.55) (end 130.5 77.95) (width 0.5) (layer "F.Cu") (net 2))
 (segment (start 121.92 77.58) (end 123.21048 76.28952) (width 0.5) (layer "F.Cu") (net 2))
 (segment (start 123.21048 76.28952) (end 129.76048 76.28952) (width 0.5) (layer "F.Cu") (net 2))
 (segment (start 126.5 72.5) (end 127.54952 73.54952) (width 0.5) (layer "F.Cu") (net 8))
 (segment (start 138.49952 73.54952) (end 139.95 75) (width 0.5) (layer "F.Cu") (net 8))
 (segment (start 127.54952 73.54952) (end 138.49952 73.54952) (width 0.5) (layer "F.Cu") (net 8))
 (segment (start 143 86) (end 143 88.5) (width 0.5) (layer "F.Cu") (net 13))
 (segment (start 141 90.5) (end 118 90.5) (width 0.5) (layer "F.Cu") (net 13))
 (segment (start 144.800481 84.199519) (end 143 86) (width 0.5) (layer "F.Cu") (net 13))
 (segment (start 116.5 89) (end 116.5 77.42) (width 0.5) (layer "F.Cu") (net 13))
 (segment (start 148.05 82) (end 148.05 82.43927) (width 0.5) (layer "F.Cu") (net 13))
 (segment (start 146.289751 84.199519) (end 144.800481 84.199519) (width 0.5) (layer "F.Cu") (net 13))
 (segment (start 118 90.5) (end 116.5 89) (width 0.5) (layer "F.Cu") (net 13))
 (segment (start 143 88.5) (end 141 90.5) (width 0.5) (layer "F.Cu") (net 13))
 (segment (start 116.5 77.42) (end 118.88 75.04) (width 0.5) (layer "F.Cu") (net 13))
 (segment (start 148.05 82.43927) (end 146.289751 84.199519) (width 0.5) (layer "F.Cu") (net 13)))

